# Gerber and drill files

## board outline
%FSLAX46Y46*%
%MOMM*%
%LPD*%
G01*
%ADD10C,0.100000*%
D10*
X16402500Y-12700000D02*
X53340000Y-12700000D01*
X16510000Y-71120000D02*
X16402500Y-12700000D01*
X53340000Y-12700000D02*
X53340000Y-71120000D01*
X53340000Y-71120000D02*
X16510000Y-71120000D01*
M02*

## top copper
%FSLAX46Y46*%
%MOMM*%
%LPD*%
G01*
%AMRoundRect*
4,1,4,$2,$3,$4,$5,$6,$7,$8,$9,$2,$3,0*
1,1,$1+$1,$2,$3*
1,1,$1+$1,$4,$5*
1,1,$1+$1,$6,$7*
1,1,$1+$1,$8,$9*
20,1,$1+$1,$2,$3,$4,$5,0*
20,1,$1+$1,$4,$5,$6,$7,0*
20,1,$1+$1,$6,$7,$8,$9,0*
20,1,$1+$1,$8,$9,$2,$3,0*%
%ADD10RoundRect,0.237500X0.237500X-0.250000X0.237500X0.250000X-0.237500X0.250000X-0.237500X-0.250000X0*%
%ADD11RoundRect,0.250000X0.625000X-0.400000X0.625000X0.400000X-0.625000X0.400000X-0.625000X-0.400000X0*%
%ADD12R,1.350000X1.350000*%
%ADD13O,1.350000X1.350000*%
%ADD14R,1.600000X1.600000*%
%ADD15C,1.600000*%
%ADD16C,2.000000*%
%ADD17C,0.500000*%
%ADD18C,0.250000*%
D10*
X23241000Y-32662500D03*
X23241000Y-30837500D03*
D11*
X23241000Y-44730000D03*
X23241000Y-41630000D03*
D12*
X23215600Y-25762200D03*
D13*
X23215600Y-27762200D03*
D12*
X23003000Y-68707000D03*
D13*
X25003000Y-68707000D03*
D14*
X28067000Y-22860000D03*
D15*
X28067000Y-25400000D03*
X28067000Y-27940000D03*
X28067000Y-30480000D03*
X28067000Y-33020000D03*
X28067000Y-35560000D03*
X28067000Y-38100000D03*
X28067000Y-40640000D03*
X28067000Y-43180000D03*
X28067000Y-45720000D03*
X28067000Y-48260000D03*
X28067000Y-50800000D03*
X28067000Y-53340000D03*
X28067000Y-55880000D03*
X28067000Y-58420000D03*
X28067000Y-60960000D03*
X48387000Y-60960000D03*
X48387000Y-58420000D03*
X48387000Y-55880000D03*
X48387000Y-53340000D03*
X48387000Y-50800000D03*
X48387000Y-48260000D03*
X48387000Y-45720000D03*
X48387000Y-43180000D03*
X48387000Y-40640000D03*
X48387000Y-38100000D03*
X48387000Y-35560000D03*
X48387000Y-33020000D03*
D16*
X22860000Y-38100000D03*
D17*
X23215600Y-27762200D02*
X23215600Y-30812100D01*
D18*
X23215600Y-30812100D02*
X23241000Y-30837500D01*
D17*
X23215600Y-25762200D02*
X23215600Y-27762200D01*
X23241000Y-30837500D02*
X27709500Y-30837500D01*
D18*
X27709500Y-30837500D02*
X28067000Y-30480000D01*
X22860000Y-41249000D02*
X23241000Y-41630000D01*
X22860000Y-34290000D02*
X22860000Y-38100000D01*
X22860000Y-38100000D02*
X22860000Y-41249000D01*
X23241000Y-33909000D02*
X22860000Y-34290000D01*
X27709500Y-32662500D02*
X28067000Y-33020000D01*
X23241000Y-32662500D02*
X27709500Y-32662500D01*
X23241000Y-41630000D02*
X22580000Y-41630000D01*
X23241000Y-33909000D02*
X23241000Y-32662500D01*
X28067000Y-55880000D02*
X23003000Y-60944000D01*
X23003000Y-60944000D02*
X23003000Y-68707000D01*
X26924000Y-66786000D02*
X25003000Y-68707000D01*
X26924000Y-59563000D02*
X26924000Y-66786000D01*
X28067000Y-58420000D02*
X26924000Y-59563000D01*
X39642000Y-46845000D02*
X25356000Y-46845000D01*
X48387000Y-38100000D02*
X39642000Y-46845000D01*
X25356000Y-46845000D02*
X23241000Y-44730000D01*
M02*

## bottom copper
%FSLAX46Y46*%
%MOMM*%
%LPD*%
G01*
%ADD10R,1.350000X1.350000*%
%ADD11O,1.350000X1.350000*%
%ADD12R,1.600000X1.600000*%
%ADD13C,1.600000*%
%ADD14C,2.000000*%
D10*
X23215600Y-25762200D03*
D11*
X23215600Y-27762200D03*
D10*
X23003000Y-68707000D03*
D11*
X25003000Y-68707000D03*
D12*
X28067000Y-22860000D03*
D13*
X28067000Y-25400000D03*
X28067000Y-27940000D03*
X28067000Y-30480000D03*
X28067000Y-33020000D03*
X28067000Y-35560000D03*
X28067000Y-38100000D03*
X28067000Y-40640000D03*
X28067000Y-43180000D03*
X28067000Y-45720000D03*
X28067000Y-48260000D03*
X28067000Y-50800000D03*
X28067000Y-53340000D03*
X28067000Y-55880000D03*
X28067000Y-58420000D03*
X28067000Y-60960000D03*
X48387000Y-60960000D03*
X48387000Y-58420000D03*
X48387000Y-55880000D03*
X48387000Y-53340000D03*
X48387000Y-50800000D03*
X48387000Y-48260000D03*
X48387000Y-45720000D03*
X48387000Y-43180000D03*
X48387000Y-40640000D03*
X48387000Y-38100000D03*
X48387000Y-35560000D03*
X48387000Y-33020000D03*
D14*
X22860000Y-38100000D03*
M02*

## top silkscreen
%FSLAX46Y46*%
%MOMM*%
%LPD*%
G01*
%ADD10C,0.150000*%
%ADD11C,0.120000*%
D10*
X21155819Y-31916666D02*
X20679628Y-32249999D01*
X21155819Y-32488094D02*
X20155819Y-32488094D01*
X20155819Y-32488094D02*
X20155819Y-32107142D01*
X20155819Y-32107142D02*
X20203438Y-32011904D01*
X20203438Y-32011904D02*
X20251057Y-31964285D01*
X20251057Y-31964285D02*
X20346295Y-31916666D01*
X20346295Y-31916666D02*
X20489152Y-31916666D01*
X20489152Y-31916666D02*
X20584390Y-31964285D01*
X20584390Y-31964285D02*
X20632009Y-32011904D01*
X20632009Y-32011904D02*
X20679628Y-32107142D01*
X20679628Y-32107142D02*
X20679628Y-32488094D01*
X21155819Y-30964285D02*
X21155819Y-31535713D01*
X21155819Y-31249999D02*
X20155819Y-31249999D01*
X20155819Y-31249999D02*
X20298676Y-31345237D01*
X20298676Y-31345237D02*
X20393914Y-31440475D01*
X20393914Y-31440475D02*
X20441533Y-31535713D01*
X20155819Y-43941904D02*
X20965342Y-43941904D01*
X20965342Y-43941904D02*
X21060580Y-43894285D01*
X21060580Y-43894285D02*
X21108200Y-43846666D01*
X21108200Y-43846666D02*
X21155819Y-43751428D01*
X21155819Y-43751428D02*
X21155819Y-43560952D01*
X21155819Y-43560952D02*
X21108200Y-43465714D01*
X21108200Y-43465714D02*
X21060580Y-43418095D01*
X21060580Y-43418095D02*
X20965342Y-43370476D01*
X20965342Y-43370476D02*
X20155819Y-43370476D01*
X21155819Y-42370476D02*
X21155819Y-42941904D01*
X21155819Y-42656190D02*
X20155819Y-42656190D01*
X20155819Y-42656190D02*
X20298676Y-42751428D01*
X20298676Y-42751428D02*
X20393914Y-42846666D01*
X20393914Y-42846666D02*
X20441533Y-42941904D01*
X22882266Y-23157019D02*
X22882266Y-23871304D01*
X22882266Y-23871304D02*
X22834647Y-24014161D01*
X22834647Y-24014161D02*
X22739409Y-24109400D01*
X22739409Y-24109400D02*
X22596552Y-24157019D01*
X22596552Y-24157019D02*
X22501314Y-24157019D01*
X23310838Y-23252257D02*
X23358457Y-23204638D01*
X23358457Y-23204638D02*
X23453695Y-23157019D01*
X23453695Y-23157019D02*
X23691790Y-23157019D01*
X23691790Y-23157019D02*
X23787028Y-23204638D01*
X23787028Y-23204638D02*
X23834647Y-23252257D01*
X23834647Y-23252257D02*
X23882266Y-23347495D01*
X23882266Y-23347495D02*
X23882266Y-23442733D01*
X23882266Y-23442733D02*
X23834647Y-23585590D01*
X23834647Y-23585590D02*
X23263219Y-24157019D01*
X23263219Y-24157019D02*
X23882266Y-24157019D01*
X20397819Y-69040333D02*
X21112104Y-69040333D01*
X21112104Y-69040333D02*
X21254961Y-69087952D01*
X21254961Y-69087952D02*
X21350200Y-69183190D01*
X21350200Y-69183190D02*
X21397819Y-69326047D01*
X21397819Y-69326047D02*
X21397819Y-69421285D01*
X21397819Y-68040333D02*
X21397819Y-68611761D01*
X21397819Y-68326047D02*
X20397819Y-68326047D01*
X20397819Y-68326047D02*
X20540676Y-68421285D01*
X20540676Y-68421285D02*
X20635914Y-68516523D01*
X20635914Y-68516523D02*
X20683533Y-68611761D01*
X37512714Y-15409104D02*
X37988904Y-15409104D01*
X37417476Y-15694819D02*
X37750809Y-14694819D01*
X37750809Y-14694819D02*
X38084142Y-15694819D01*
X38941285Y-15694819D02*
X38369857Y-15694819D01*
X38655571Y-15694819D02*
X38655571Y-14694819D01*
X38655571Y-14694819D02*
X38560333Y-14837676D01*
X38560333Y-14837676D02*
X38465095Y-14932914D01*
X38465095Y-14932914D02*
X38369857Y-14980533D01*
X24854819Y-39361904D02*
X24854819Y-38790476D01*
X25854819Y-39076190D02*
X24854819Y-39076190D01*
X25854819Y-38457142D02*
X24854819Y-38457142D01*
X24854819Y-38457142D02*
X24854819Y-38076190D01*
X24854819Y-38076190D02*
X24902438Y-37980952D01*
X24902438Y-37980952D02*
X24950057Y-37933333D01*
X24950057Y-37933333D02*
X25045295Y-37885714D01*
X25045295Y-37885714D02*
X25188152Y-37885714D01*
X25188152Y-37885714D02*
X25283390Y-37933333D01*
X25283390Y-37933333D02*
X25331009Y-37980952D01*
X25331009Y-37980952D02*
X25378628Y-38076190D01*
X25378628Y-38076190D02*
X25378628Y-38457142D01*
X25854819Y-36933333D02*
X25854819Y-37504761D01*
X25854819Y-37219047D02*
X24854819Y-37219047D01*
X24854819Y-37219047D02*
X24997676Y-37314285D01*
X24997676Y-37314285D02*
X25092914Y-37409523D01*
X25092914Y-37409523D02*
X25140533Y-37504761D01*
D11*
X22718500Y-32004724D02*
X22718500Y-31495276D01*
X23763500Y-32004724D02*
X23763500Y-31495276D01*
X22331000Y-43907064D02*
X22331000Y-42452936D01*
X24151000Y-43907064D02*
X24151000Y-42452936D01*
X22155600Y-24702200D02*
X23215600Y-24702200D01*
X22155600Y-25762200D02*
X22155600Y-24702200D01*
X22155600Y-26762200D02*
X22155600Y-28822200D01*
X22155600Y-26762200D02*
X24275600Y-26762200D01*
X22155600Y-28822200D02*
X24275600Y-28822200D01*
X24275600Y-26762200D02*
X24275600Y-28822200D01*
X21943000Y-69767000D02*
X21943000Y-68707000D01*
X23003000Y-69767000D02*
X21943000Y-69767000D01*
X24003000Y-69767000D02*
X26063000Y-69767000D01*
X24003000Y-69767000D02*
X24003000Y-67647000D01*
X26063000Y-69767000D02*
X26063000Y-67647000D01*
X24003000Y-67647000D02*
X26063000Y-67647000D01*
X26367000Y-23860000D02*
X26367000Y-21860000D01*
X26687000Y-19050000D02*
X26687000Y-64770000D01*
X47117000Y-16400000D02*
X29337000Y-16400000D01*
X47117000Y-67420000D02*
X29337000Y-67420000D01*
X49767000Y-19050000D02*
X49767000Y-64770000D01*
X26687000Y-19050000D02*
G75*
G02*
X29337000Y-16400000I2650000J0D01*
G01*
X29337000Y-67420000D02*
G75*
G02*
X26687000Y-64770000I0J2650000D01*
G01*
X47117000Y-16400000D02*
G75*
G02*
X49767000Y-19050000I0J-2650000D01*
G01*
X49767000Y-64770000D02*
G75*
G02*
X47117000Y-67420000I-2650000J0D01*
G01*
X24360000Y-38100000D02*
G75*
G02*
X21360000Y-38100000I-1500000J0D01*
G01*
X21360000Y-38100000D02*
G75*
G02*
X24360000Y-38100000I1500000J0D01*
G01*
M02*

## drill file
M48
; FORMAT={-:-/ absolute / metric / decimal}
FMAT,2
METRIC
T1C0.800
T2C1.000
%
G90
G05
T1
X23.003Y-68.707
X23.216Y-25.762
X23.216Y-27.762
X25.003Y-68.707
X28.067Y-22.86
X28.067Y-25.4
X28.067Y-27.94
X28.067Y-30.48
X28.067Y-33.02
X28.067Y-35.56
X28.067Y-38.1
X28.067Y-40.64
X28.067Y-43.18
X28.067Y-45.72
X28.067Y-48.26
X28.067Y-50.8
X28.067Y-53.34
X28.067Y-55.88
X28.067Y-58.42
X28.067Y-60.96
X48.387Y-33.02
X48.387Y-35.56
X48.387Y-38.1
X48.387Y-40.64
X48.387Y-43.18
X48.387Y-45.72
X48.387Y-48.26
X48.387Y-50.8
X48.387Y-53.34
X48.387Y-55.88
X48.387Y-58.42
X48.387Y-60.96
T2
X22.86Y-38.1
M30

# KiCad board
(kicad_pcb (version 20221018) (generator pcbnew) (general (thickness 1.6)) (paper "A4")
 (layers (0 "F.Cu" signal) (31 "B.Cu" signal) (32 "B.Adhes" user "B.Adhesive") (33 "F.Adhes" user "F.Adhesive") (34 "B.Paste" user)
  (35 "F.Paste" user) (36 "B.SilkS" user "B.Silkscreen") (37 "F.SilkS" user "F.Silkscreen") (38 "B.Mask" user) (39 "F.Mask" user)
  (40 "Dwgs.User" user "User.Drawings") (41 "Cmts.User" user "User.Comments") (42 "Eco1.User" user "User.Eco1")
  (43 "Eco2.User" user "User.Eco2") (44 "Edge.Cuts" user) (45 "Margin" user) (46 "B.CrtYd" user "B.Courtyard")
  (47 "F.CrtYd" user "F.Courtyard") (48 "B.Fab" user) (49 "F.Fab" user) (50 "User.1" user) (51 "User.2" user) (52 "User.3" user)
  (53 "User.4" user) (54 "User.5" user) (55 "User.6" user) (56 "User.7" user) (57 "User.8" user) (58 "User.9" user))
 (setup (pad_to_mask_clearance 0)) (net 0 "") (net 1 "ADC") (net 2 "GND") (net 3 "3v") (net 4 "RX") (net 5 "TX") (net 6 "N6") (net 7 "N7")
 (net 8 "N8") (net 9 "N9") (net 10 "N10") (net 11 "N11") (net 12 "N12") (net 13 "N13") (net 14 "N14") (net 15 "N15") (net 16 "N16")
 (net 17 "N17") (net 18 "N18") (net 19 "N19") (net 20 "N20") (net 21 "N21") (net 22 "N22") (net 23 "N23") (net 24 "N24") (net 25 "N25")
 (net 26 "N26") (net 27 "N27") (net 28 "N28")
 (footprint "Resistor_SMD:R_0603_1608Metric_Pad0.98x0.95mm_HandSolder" (layer "F.Cu") (at 23.241 31.75 90)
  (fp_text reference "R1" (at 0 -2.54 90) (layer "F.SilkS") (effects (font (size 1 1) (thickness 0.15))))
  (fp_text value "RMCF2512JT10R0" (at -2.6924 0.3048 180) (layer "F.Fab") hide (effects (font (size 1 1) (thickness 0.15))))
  (fp_line (start -0.254724 -0.5225) (end 0.254724 -0.5225) (stroke (width 0.12) (type solid)) (layer "F.SilkS"))
  (fp_line (start -0.254724 0.5225) (end 0.254724 0.5225) (stroke (width 0.12) (type solid)) (layer "F.SilkS"))
  (pad "1" smd roundrect (at -0.9125 0 90) (size 0.975 0.95) (layers "F.Cu" "F.Paste" "F.Mask") (roundrect_rratio 0.25) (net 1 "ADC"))
  (pad "2" smd roundrect (at 0.9125 0 90) (size 0.975 0.95) (layers "F.Cu" "F.Paste" "F.Mask") (roundrect_rratio 0.25) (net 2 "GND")))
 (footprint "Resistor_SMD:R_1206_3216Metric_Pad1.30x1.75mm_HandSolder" (layer "F.Cu") (at 23.241 43.18 90)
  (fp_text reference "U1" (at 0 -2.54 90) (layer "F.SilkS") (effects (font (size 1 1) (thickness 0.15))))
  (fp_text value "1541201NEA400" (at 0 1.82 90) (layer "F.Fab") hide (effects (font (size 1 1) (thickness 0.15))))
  (fp_line (start -0.727064 -0.91) (end 0.727064 -0.91) (stroke (width 0.12) (type solid)) (layer "F.SilkS"))
  (fp_line (start -0.727064 0.91) (end 0.727064 0.91) (stroke (width 0.12) (type solid)) (layer "F.SilkS"))
  (pad "1" smd roundrect (at -1.55 0 90) (size 1.3 1.75) (layers "F.Cu" "F.Paste" "F.Mask") (roundrect_rratio 0.1923076923) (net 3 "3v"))
  (pad "2" smd roundrect (at 1.55 0 90) (size 1.3 1.75) (layers "F.Cu" "F.Paste" "F.Mask") (roundrect_rratio 0.1923076923) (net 1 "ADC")))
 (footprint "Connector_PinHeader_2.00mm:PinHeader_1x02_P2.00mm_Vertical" (layer "F.Cu") (at 23.2156 25.7622)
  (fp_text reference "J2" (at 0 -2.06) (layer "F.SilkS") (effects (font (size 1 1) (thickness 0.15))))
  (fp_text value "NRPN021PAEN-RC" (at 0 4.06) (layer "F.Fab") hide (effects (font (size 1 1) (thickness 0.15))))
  (fp_line (start -1.06 -1.06) (end 0 -1.06) (stroke (width 0.12) (type solid)) (layer "F.SilkS"))
  (fp_line (start -1.06 0) (end -1.06 -1.06) (stroke (width 0.12) (type solid)) (layer "F.SilkS"))
  (fp_line (start -1.06 1) (end -1.06 3.06) (stroke (width 0.12) (type solid)) (layer "F.SilkS"))
  (fp_line (start -1.06 1) (end 1.06 1) (stroke (width 0.12) (type solid)) (layer "F.SilkS"))
  (fp_line (start -1.06 3.06) (end 1.06 3.06) (stroke (width 0.12) (type solid)) (layer "F.SilkS"))
  (fp_line (start 1.06 1) (end 1.06 3.06) (stroke (width 0.12) (type solid)) (layer "F.SilkS"))
  (pad "1" thru_hole rect (at 0 0) (size 1.35 1.35) (drill 0.8) (layers "*.Cu" "*.Mask") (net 2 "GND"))
  (pad "2" thru_hole oval (at 0 2) (size 1.35 1.35) (drill 0.8) (layers "*.Cu" "*.Mask") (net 2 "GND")))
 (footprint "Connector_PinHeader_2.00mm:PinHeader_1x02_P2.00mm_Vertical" (layer "F.Cu") (at 23.003 68.707 90)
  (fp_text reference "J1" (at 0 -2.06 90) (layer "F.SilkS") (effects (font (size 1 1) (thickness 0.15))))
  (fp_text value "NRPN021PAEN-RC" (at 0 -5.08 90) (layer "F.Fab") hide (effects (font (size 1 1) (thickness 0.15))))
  (fp_line (start -1.06 -1.06) (end 0 -1.06) (stroke (width 0.12) (type solid)) (layer "F.SilkS"))
  (fp_line (start -1.06 0) (end -1.06 -1.06) (stroke (width 0.12) (type solid)) (layer "F.SilkS"))
  (fp_line (start -1.06 1) (end -1.06 3.06) (stroke (width 0.12) (type solid)) (layer "F.SilkS"))
  (fp_line (start -1.06 1) (end 1.06 1) (stroke (width 0.12) (type solid)) (layer "F.SilkS"))
  (fp_line (start -1.06 3.06) (end 1.06 3.06) (stroke (width 0.12) (type solid)) (layer "F.SilkS"))
  (fp_line (start 1.06 1) (end 1.06 3.06) (stroke (width 0.12) (type solid)) (layer "F.SilkS"))
  (pad "1" thru_hole rect (at 0 0 90) (size 1.35 1.35) (drill 0.8) (layers "*.Cu" "*.Mask") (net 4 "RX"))
  (pad "2" thru_hole oval (at 0 2 90) (size 1.35 1.35) (drill 0.8) (layers "*.Cu" "*.Mask") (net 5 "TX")))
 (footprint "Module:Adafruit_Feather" (layer "F.Cu") (at 28.067 22.86)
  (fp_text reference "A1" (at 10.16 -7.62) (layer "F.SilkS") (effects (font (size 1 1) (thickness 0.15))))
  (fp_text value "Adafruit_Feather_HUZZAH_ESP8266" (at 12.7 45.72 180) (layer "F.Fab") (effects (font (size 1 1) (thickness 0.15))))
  (fp_line (start -1.7 1) (end -1.7 -1) (stroke (width 0.12) (type solid)) (layer "F.SilkS"))
  (fp_line (start -1.38 -3.81) (end -1.38 41.91) (stroke (width 0.12) (type solid)) (layer "F.SilkS"))
  (fp_line (start 19.05 -6.46) (end 1.27 -6.46) (stroke (width 0.12) (type solid)) (layer "F.SilkS"))
  (fp_line (start 19.05 44.56) (end 1.27 44.56) (stroke (width 0.12) (type solid)) (layer "F.SilkS"))
  (fp_line (start 21.7 -3.81) (end 21.7 41.91) (stroke (width 0.12) (type solid)) (layer "F.SilkS"))
  (fp_arc (start -1.38 -3.81) (mid -0.603833 -5.683833) (end 1.27 -6.46) (stroke (width 0.12) (type solid)) (layer "F.SilkS"))
  (fp_arc (start 1.27 44.56) (mid -0.603833 43.783833) (end -1.38 41.91) (stroke (width 0.12) (type solid)) (layer "F.SilkS"))
  (fp_arc (start 19.05 -6.46) (mid 20.923833 -5.683833) (end 21.7 -3.81) (stroke (width 0.12) (type solid)) (layer "F.SilkS"))
  (fp_arc (start 21.7 41.91) (mid 20.923833 43.783833) (end 19.05 44.56) (stroke (width 0.12) (type solid)) (layer "F.SilkS"))
  (pad "1" thru_hole rect (at 0 0 180) (size 1.6 1.6) (drill 0.8) (layers "*.Cu" "*.Mask") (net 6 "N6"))
  (pad "2" thru_hole circle (at 0 2.54 180) (size 1.6 1.6) (drill 0.8) (layers "*.Cu" "*.Mask") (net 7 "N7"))
  (pad "3" thru_hole circle (at 0 5.08 180) (size 1.6 1.6) (drill 0.8) (layers "*.Cu" "*.Mask") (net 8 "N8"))
  (pad "4" thru_hole circle (at 0 7.62 180) (size 1.6 1.6) (drill 0.8) (layers "*.Cu" "*.Mask") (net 2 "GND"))
  (pad "5" thru_hole circle (at 0 10.16 180) (size 1.6 1.6) (drill 0.8) (layers "*.Cu" "*.Mask") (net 1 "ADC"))
  (pad "6" thru_hole circle (at 0 12.7 180) (size 1.6 1.6) (drill 0.8) (layers "*.Cu" "*.Mask") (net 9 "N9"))
  (pad "7" thru_hole circle (at 0 15.24 180) (size 1.6 1.6) (drill 0.8) (layers "*.Cu" "*.Mask") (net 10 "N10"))
  (pad "8" thru_hole circle (at 0 17.78 180) (size 1.6 1.6) (drill 0.8) (layers "*.Cu" "*.Mask") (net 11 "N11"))
  (pad "9" thru_hole circle (at 0 20.32 180) (size 1.6 1.6) (drill 0.8) (layers "*.Cu" "*.Mask") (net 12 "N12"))
  (pad "10" thru_hole circle (at 0 22.86 180) (size 1.6 1.6) (drill 0.8) (layers "*.Cu" "*.Mask") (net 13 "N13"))
  (pad "11" thru_hole circle (at 0 25.4 180) (size 1.6 1.6) (drill 0.8) (layers "*.Cu" "*.Mask") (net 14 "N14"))
  (pad "12" thru_hole circle (at 0 27.94 180) (size 1.6 1.6) (drill 0.8) (layers "*.Cu" "*.Mask") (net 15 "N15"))
  (pad "13" thru_hole circle (at 0 30.48 180) (size 1.6 1.6) (drill 0.8) (layers "*.Cu" "*.Mask") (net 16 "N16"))
  (pad "14" thru_hole circle (at 0 33.02 180) (size 1.6 1.6) (drill 0.8) (layers "*.Cu" "*.Mask") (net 4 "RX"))
  (pad "15" thru_hole circle (at 0 35.56 180) (size 1.6 1.6) (drill 0.8) (layers "*.Cu" "*.Mask") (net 5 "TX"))
  (pad "16" thru_hole circle (at 0 38.1 180) (size 1.6 1.6) (drill 0.8) (layers "*.Cu" "*.Mask") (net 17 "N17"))
  (pad "17" thru_hole circle (at 20.32 38.1 180) (size 1.6 1.6) (drill 0.8) (layers "*.Cu" "*.Mask") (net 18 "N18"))
  (pad "18" thru_hole circle (at 20.32 35.56 180) (size 1.6 1.6) (drill 0.8) (layers "*.Cu" "*.Mask") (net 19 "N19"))
  (pad "19" thru_hole circle (at 20.32 33.02 180) (size 1.6 1.6) (drill 0.8) (layers "*.Cu" "*.Mask") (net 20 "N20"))
  (pad "20" thru_hole circle (at 20.32 30.48 180) (size 1.6 1.6) (drill 0.8) (layers "*.Cu" "*.Mask") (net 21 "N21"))
  (pad "21" thru_hole circle (at 20.32 27.94 180) (size 1.6 1.6) (drill 0.8) (layers "*.Cu" "*.Mask") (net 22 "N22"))
  (pad "22" thru_hole circle (at 20.32 25.4 180) (size 1.6 1.6) (drill 0.8) (layers "*.Cu" "*.Mask") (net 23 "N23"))
  (pad "23" thru_hole circle (at 20.32 22.86 180) (size 1.6 1.6) (drill 0.8) (layers "*.Cu" "*.Mask") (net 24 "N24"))
  (pad "24" thru_hole circle (at 20.32 20.32 180) (size 1.6 1.6) (drill 0.8) (layers "*.Cu" "*.Mask") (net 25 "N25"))
  (pad "25" thru_hole circle (at 20.32 17.78 180) (size 1.6 1.6) (drill 0.8) (layers "*.Cu" "*.Mask") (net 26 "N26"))
  (pad "26" thru_hole circle (at 20.32 15.24 180) (size 1.6 1.6) (drill 0.8) (layers "*.Cu" "*.Mask") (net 3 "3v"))
  (pad "27" thru_hole circle (at 20.32 12.7 180) (size 1.6 1.6) (drill 0.8) (layers "*.Cu" "*.Mask") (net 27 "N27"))
  (pad "28" thru_hole circle (at 20.32 10.16 180) (size 1.6 1.6) (drill 0.8) (layers "*.Cu" "*.Mask") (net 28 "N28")))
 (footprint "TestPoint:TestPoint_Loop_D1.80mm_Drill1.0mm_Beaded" (layer "F.Cu") (at 22.86 38.1)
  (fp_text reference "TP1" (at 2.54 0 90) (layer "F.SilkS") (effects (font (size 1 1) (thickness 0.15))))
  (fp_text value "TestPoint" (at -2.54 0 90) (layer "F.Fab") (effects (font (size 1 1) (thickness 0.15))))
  (fp_circle (center 0 0) (end 1.5 0) (stroke (width 0.12) (type solid)) (fill none) (layer "F.SilkS"))
  (pad "1" thru_hole circle (at 0 0) (size 2 2) (drill 1) (layers "*.Cu" "*.Mask") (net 1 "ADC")))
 (gr_line (start 16.4025 12.7) (end 53.34 12.7) (stroke (width 0.1) (type default)) (layer "Edge.Cuts"))
 (gr_line (start 16.51 71.12) (end 16.4025 12.7) (stroke (width 0.1) (type default)) (layer "Edge.Cuts"))
 (gr_line (start 53.34 12.7) (end 53.34 71.12) (stroke (width 0.1) (type default)) (layer "Edge.Cuts"))
 (gr_line (start 53.34 71.12) (end 16.51 71.12) (stroke (width 0.1) (type default)) (layer "Edge.Cuts"))
 (segment (start 23.2156 27.7622) (end 23.2156 30.8121) (width 0.5) (layer "F.Cu") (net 2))
 (segment (start 23.2156 30.8121) (end 23.241 30.8375) (width 0.25) (layer "F.Cu") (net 2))
 (segment (start 23.2156 25.7622) (end 23.2156 27.7622) (width 0.5) (layer "F.Cu") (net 2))
 (segment (start 23.241 30.8375) (end 27.7095 30.8375) (width 0.5) (layer "F.Cu") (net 2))
 (segment (start 27.7095 30.8375) (end 28.067 30.48) (width 0.25) (layer "F.Cu") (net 2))
 (segment (start 22.86 41.249) (end 23.241 41.63) (width 0.25) (layer "F.Cu") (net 1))
 (segment (start 22.86 34.29) (end 22.86 38.1) (width 0.25) (layer "F.Cu") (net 1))
 (segment (start 22.86 38.1) (end 22.86 41.249) (width 0.25) (layer "F.Cu") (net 1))
 (segment (start 23.241 33.909) (end 22.86 34.29) (width 0.25) (layer "F.Cu") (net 1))
 (segment (start 27.7095 32.6625) (end 28.067 33.02) (width 0.25) (layer "F.Cu") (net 1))
 (segment (start 23.241 32.6625) (end 27.7095 32.6625) (width 0.25) (layer "F.Cu") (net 1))
 (segment (start 23.241 41.63) (end 22.58 41.63) (width 0.25) (layer "F.Cu") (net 1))
 (segment (start 23.241 33.909) (end 23.241 32.6625) (width 0.25) (layer "F.Cu") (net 1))
 (segment (start 28.067 55.88) (end 23.003 60.944) (width 0.25) (layer "F.Cu") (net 4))
 (segment (start 23.003 60.944) (end 23.003 68.707) (width 0.25) (layer "F.Cu") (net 4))
 (segment (start 26.924 66.786) (end 25.003 68.707) (width 0.25) (layer "F.Cu") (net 5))
 (segment (start 26.924 59.563) (end 26.924 66.786) (width 0.25) (layer "F.Cu") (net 5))
 (segment (start 28.067 58.42) (end 26.924 59.563) (width 0.25) (layer "F.Cu") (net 5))
 (segment (start 39.642 46.845) (end 25.356 46.845) (width 0.25) (layer "F.Cu") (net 3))
 (segment (start 48.387 38.1) (end 39.642 46.845) (width 0.25) (layer "F.Cu") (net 3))
 (segment (start 25.356 46.845) (end 23.241 44.73) (width 0.25) (layer "F.Cu") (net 3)))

